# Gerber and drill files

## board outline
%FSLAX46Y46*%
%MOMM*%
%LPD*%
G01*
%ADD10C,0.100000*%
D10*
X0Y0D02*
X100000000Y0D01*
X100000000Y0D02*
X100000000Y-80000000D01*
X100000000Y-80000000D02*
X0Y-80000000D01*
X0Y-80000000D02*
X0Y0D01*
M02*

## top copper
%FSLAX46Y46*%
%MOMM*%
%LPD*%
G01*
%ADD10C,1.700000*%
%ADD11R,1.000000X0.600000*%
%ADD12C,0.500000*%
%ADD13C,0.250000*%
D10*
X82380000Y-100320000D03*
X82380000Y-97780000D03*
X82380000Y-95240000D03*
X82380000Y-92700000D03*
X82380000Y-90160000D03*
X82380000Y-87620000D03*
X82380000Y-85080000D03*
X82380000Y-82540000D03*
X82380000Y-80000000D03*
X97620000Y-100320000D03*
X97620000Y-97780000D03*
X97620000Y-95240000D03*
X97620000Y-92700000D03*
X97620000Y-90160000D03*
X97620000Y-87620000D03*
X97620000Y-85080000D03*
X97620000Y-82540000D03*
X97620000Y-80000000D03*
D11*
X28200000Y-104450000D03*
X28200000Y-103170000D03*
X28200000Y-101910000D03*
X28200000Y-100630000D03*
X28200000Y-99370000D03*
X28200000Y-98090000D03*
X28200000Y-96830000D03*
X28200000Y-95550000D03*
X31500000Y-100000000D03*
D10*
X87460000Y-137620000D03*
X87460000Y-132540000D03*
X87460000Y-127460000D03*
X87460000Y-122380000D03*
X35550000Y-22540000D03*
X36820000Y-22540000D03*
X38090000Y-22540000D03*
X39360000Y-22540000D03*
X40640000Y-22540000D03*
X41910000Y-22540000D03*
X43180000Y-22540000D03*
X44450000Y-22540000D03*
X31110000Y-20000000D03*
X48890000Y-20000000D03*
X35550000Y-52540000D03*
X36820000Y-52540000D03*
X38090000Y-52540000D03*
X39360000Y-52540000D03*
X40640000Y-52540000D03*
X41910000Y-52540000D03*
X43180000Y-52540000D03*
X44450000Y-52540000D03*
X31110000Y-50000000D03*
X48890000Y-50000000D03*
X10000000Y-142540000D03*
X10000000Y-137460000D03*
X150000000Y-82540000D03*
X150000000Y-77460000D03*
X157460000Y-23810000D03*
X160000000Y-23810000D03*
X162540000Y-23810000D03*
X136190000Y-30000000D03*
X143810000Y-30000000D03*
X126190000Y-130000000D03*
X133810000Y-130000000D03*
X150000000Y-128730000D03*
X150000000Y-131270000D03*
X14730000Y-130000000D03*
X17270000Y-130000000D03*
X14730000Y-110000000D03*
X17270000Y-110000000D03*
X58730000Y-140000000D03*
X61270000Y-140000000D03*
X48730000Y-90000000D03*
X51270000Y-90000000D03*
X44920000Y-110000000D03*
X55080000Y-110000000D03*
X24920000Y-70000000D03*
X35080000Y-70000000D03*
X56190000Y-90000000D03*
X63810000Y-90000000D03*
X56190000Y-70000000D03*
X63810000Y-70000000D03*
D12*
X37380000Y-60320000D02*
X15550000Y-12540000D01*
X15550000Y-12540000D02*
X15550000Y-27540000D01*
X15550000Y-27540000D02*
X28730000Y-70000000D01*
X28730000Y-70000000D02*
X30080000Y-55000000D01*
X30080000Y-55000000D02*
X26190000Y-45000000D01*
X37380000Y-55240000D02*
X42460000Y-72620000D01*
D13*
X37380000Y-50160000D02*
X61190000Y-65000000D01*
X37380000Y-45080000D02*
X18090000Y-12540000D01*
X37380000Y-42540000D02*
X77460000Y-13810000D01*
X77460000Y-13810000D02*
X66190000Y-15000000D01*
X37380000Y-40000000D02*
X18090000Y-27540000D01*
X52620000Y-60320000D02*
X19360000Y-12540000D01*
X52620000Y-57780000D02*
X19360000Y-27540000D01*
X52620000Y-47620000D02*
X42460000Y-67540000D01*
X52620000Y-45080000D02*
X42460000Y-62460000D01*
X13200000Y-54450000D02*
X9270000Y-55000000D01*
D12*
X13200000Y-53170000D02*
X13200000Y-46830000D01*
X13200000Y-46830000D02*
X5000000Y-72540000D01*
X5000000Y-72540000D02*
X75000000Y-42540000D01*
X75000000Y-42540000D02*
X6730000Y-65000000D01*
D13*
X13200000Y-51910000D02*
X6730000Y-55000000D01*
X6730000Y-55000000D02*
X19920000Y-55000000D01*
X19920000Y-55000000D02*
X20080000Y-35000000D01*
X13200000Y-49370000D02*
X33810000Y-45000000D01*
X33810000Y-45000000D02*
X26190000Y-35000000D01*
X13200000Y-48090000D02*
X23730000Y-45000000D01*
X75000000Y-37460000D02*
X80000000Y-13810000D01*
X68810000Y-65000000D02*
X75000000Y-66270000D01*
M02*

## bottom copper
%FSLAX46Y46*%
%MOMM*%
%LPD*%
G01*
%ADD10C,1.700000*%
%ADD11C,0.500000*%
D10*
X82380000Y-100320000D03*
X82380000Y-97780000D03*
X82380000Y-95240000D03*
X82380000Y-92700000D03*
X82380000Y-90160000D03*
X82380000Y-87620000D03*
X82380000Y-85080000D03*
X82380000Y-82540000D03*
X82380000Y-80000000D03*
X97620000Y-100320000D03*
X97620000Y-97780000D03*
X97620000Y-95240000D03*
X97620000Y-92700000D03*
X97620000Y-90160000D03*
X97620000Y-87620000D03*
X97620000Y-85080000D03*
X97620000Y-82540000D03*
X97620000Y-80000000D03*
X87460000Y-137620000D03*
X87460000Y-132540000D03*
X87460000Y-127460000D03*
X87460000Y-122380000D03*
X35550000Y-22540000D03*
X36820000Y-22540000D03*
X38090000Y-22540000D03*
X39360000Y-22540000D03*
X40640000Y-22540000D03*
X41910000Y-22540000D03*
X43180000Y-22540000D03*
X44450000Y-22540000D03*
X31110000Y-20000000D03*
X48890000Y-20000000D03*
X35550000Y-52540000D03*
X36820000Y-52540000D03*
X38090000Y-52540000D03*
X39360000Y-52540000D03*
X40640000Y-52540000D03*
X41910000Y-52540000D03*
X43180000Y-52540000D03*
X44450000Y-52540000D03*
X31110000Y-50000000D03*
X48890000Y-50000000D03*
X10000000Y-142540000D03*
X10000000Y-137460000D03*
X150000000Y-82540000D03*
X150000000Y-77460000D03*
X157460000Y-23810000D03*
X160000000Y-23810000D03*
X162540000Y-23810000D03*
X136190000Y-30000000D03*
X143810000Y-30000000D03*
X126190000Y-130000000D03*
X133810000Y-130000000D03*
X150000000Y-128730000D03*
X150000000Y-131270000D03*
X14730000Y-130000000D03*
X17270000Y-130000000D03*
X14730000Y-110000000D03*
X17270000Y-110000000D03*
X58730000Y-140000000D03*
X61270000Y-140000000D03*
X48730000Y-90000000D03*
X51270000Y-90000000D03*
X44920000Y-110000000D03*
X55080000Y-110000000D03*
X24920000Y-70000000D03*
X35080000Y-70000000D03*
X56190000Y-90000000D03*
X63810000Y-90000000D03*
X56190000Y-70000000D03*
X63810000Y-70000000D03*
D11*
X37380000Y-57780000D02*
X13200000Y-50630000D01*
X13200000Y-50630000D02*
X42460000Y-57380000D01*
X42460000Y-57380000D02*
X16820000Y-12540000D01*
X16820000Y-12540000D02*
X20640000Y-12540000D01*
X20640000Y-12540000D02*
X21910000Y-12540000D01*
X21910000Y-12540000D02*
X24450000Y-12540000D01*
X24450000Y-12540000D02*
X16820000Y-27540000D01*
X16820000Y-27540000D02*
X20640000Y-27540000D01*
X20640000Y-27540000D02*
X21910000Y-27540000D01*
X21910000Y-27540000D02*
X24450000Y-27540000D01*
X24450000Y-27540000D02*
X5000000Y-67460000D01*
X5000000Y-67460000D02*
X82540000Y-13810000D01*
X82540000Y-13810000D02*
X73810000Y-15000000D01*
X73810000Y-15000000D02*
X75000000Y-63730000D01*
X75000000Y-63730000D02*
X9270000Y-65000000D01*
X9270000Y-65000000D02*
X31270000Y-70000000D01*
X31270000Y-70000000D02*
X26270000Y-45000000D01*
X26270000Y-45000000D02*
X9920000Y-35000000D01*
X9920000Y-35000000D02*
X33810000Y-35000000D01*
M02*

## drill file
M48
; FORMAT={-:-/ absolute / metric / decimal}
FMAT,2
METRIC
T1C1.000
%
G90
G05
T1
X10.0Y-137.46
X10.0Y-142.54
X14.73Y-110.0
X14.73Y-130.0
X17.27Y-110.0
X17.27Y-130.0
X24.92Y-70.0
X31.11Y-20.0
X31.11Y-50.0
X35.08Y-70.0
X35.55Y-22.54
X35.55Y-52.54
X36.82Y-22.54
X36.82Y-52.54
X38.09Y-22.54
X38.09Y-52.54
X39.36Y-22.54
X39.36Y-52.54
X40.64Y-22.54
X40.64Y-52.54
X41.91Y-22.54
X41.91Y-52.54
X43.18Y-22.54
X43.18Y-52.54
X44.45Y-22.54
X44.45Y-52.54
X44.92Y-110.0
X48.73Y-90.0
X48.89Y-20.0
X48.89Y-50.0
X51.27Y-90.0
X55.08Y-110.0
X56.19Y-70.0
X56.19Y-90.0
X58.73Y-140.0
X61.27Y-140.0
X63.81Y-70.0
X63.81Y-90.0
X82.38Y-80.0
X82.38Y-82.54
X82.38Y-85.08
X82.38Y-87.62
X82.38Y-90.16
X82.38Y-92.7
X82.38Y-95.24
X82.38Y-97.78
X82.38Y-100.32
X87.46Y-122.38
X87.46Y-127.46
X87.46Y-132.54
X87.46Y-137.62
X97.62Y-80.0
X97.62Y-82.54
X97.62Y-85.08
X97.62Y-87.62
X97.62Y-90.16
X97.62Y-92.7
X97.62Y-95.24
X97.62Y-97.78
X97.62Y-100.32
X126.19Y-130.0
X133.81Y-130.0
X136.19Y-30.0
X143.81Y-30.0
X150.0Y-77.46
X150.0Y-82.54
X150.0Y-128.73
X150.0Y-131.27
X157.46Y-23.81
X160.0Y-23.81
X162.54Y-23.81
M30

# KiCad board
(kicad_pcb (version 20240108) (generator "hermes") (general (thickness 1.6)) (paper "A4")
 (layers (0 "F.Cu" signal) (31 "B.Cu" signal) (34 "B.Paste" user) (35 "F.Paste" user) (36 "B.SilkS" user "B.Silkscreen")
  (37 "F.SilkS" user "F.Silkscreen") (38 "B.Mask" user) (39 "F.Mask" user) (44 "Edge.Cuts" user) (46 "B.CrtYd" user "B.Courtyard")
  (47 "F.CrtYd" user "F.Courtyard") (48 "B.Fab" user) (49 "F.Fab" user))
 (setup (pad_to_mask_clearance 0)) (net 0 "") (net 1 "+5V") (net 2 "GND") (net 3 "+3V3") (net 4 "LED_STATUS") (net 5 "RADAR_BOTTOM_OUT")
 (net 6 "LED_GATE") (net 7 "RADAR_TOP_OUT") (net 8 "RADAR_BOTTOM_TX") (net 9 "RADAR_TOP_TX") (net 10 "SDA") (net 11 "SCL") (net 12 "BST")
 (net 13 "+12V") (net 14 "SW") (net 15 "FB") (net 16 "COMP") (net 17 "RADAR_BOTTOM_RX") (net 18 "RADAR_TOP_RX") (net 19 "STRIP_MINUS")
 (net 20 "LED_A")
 (gr_line (start 0 0) (end 100 0) (stroke (width 0.1) (type default)) (layer "Edge.Cuts"))
 (gr_line (start 100 0) (end 100 80) (stroke (width 0.1) (type default)) (layer "Edge.Cuts"))
 (gr_line (start 100 80) (end 0 80) (stroke (width 0.1) (type default)) (layer "Edge.Cuts"))
 (gr_line (start 0 80) (end 0 0) (stroke (width 0.1) (type default)) (layer "Edge.Cuts"))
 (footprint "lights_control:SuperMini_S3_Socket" (layer "F.Cu") (at 45 40 0) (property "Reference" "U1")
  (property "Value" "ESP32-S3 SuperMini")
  (pad "1" thru_hole circle (at 37.38 60.32) (size 1.7 1.7) (drill 1.0) (layers "*.Cu" "*.Mask") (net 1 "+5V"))
  (pad "2" thru_hole circle (at 37.38 57.78) (size 1.7 1.7) (drill 1.0) (layers "*.Cu" "*.Mask") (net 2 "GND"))
  (pad "3" thru_hole circle (at 37.38 55.24) (size 1.7 1.7) (drill 1.0) (layers "*.Cu" "*.Mask") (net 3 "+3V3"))
  (pad "4" thru_hole circle (at 37.38 52.70) (size 1.7 1.7) (drill 1.0) (layers "*.Cu" "*.Mask"))
  (pad "5" thru_hole circle (at 37.38 50.16) (size 1.7 1.7) (drill 1.0) (layers "*.Cu" "*.Mask") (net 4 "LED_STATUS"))
  (pad "6" thru_hole circle (at 37.38 47.62) (size 1.7 1.7) (drill 1.0) (layers "*.Cu" "*.Mask"))
  (pad "7" thru_hole circle (at 37.38 45.08) (size 1.7 1.7) (drill 1.0) (layers "*.Cu" "*.Mask") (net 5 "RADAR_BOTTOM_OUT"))
  (pad "8" thru_hole circle (at 37.38 42.54) (size 1.7 1.7) (drill 1.0) (layers "*.Cu" "*.Mask") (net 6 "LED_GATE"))
  (pad "9" thru_hole circle (at 37.38 40.00) (size 1.7 1.7) (drill 1.0) (layers "*.Cu" "*.Mask") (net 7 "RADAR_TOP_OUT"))
  (pad "10" thru_hole circle (at 52.62 60.32) (size 1.7 1.7) (drill 1.0) (layers "*.Cu" "*.Mask") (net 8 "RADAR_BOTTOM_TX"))
  (pad "11" thru_hole circle (at 52.62 57.78) (size 1.7 1.7) (drill 1.0) (layers "*.Cu" "*.Mask") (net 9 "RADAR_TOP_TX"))
  (pad "12" thru_hole circle (at 52.62 55.24) (size 1.7 1.7) (drill 1.0) (layers "*.Cu" "*.Mask"))
  (pad "13" thru_hole circle (at 52.62 52.70) (size 1.7 1.7) (drill 1.0) (layers "*.Cu" "*.Mask"))
  (pad "14" thru_hole circle (at 52.62 50.16) (size 1.7 1.7) (drill 1.0) (layers "*.Cu" "*.Mask"))
  (pad "15" thru_hole circle (at 52.62 47.62) (size 1.7 1.7) (drill 1.0) (layers "*.Cu" "*.Mask") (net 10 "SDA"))
  (pad "16" thru_hole circle (at 52.62 45.08) (size 1.7 1.7) (drill 1.0) (layers "*.Cu" "*.Mask") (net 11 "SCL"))
  (pad "17" thru_hole circle (at 52.62 42.54) (size 1.7 1.7) (drill 1.0) (layers "*.Cu" "*.Mask"))
  (pad "18" thru_hole circle (at 52.62 40.00) (size 1.7 1.7) (drill 1.0) (layers "*.Cu" "*.Mask")))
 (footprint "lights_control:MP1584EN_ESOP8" (layer "F.Cu") (at 15 50 0) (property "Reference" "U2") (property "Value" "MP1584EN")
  (pad "1" smd rect (at 13.20 54.45) (size 1.0 0.6) (layers "F.Cu" "F.Paste" "F.Mask") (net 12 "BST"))
  (pad "2" smd rect (at 13.20 53.17) (size 1.0 0.6) (layers "F.Cu" "F.Paste" "F.Mask") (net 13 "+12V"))
  (pad "3" smd rect (at 13.20 51.91) (size 1.0 0.6) (layers "F.Cu" "F.Paste" "F.Mask") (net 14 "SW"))
  (pad "4" smd rect (at 13.20 50.63) (size 1.0 0.6) (layers "F.Cu" "F.Paste" "F.Mask") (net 2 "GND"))
  (pad "5" smd rect (at 13.20 49.37) (size 1.0 0.6) (layers "F.Cu" "F.Paste" "F.Mask") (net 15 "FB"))
  (pad "6" smd rect (at 13.20 48.09) (size 1.0 0.6) (layers "F.Cu" "F.Paste" "F.Mask") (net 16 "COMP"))
  (pad "7" smd rect (at 13.20 46.83) (size 1.0 0.6) (layers "F.Cu" "F.Paste" "F.Mask") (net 13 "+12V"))
  (pad "8" smd rect (at 13.20 45.55) (size 1.0 0.6) (layers "F.Cu" "F.Paste" "F.Mask"))
  (pad "9" smd rect (at 16.50 50.00) (size 1.0 0.6) (layers "F.Cu" "F.Paste" "F.Mask")))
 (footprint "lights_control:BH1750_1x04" (layer "F.Cu") (at 45 65 0) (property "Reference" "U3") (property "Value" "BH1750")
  (pad "1" thru_hole circle (at 42.46 72.62) (size 1.7 1.7) (drill 1.0) (layers "*.Cu" "*.Mask") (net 3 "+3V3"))
  (pad "2" thru_hole circle (at 42.46 67.54) (size 1.7 1.7) (drill 1.0) (layers "*.Cu" "*.Mask") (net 10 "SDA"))
  (pad "3" thru_hole circle (at 42.46 62.46) (size 1.7 1.7) (drill 1.0) (layers "*.Cu" "*.Mask") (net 11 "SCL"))
  (pad "4" thru_hole circle (at 42.46 57.38) (size 1.7 1.7) (drill 1.0) (layers "*.Cu" "*.Mask") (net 2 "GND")))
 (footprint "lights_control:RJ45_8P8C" (layer "F.Cu") (at 20 10 0) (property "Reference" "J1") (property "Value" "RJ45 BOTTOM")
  (pad "1" thru_hole circle (at 15.55 12.54) (size 1.7 1.7) (drill 1.0) (layers "*.Cu" "*.Mask") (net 1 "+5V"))
  (pad "2" thru_hole circle (at 16.82 12.54) (size 1.7 1.7) (drill 1.0) (layers "*.Cu" "*.Mask") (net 2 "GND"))
  (pad "3" thru_hole circle (at 18.09 12.54) (size 1.7 1.7) (drill 1.0) (layers "*.Cu" "*.Mask") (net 5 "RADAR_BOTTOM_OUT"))
  (pad "4" thru_hole circle (at 19.36 12.54) (size 1.7 1.7) (drill 1.0) (layers "*.Cu" "*.Mask") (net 8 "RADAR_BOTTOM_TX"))
  (pad "5" thru_hole circle (at 20.64 12.54) (size 1.7 1.7) (drill 1.0) (layers "*.Cu" "*.Mask") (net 2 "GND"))
  (pad "6" thru_hole circle (at 21.91 12.54) (size 1.7 1.7) (drill 1.0) (layers "*.Cu" "*.Mask") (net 2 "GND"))
  (pad "7" thru_hole circle (at 23.18 12.54) (size 1.7 1.7) (drill 1.0) (layers "*.Cu" "*.Mask") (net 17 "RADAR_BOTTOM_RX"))
  (pad "8" thru_hole circle (at 24.45 12.54) (size 1.7 1.7) (drill 1.0) (layers "*.Cu" "*.Mask") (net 2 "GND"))
  (pad "S1" thru_hole circle (at 11.11 10.00) (size 1.7 1.7) (drill 1.0) (layers "*.Cu" "*.Mask"))
  (pad "S2" thru_hole circle (at 28.89 10.00) (size 1.7 1.7) (drill 1.0) (layers "*.Cu" "*.Mask")))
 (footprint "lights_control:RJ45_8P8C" (layer "F.Cu") (at 20 25 0) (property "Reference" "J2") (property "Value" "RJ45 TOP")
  (pad "1" thru_hole circle (at 15.55 27.54) (size 1.7 1.7) (drill 1.0) (layers "*.Cu" "*.Mask") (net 1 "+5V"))
  (pad "2" thru_hole circle (at 16.82 27.54) (size 1.7 1.7) (drill 1.0) (layers "*.Cu" "*.Mask") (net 2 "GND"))
  (pad "3" thru_hole circle (at 18.09 27.54) (size 1.7 1.7) (drill 1.0) (layers "*.Cu" "*.Mask") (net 7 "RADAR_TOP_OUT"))
  (pad "4" thru_hole circle (at 19.36 27.54) (size 1.7 1.7) (drill 1.0) (layers "*.Cu" "*.Mask") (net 9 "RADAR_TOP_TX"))
  (pad "5" thru_hole circle (at 20.64 27.54) (size 1.7 1.7) (drill 1.0) (layers "*.Cu" "*.Mask") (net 2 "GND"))
  (pad "6" thru_hole circle (at 21.91 27.54) (size 1.7 1.7) (drill 1.0) (layers "*.Cu" "*.Mask") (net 2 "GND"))
  (pad "7" thru_hole circle (at 23.18 27.54) (size 1.7 1.7) (drill 1.0) (layers "*.Cu" "*.Mask") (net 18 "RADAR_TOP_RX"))
  (pad "8" thru_hole circle (at 24.45 27.54) (size 1.7 1.7) (drill 1.0) (layers "*.Cu" "*.Mask") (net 2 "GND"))
  (pad "S1" thru_hole circle (at 11.11 25.00) (size 1.7 1.7) (drill 1.0) (layers "*.Cu" "*.Mask"))
  (pad "S2" thru_hole circle (at 28.89 25.00) (size 1.7 1.7) (drill 1.0) (layers "*.Cu" "*.Mask")))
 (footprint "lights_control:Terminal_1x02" (layer "F.Cu") (at 5 70 0) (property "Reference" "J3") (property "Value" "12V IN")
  (pad "1" thru_hole circle (at 5.00 72.54) (size 1.7 1.7) (drill 1.0) (layers "*.Cu" "*.Mask") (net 13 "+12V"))
  (pad "2" thru_hole circle (at 5.00 67.46) (size 1.7 1.7) (drill 1.0) (layers "*.Cu" "*.Mask") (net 2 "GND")))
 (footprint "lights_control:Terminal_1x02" (layer "F.Cu") (at 75 40 0) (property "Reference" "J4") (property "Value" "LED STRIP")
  (pad "1" thru_hole circle (at 75.00 42.54) (size 1.7 1.7) (drill 1.0) (layers "*.Cu" "*.Mask") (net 13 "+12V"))
  (pad "2" thru_hole circle (at 75.00 37.46) (size 1.7 1.7) (drill 1.0) (layers "*.Cu" "*.Mask") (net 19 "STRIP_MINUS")))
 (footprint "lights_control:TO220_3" (layer "F.Cu") (at 80 10 0) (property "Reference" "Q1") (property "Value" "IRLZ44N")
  (pad "1" thru_hole circle (at 77.46 13.81) (size 1.7 1.7) (drill 1.0) (layers "*.Cu" "*.Mask") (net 6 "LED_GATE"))
  (pad "2" thru_hole circle (at 80.00 13.81) (size 1.7 1.7) (drill 1.0) (layers "*.Cu" "*.Mask") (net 19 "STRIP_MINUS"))
  (pad "3" thru_hole circle (at 82.54 13.81) (size 1.7 1.7) (drill 1.0) (layers "*.Cu" "*.Mask") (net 2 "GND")))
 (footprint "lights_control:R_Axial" (layer "F.Cu") (at 70 15 0) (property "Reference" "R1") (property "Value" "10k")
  (pad "1" thru_hole circle (at 66.19 15.00) (size 1.7 1.7) (drill 1.0) (layers "*.Cu" "*.Mask") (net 6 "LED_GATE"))
  (pad "2" thru_hole circle (at 73.81 15.00) (size 1.7 1.7) (drill 1.0) (layers "*.Cu" "*.Mask") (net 2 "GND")))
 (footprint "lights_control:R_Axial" (layer "F.Cu") (at 65 65 0) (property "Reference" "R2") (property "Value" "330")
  (pad "1" thru_hole circle (at 61.19 65.00) (size 1.7 1.7) (drill 1.0) (layers "*.Cu" "*.Mask") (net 4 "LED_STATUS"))
  (pad "2" thru_hole circle (at 68.81 65.00) (size 1.7 1.7) (drill 1.0) (layers "*.Cu" "*.Mask") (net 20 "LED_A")))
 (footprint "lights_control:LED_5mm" (layer "F.Cu") (at 75 65 0) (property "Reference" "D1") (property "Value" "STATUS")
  (pad "1" thru_hole circle (at 75.00 63.73) (size 1.7 1.7) (drill 1.0) (layers "*.Cu" "*.Mask") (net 2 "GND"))
  (pad "2" thru_hole circle (at 75.00 66.27) (size 1.7 1.7) (drill 1.0) (layers "*.Cu" "*.Mask") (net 20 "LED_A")))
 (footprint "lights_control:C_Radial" (layer "F.Cu") (at 8 65 0) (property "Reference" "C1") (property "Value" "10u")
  (pad "1" thru_hole circle (at 6.73 65.00) (size 1.7 1.7) (drill 1.0) (layers "*.Cu" "*.Mask") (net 13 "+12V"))
  (pad "2" thru_hole circle (at 9.27 65.00) (size 1.7 1.7) (drill 1.0) (layers "*.Cu" "*.Mask") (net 2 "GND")))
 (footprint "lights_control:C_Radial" (layer "F.Cu") (at 8 55 0) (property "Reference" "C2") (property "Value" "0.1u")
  (pad "1" thru_hole circle (at 6.73 55.00) (size 1.7 1.7) (drill 1.0) (layers "*.Cu" "*.Mask") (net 14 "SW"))
  (pad "2" thru_hole circle (at 9.27 55.00) (size 1.7 1.7) (drill 1.0) (layers "*.Cu" "*.Mask") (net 12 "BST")))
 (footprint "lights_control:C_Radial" (layer "F.Cu") (at 30 70 0) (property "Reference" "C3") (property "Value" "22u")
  (pad "1" thru_hole circle (at 28.73 70.00) (size 1.7 1.7) (drill 1.0) (layers "*.Cu" "*.Mask") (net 1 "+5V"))
  (pad "2" thru_hole circle (at 31.27 70.00) (size 1.7 1.7) (drill 1.0) (layers "*.Cu" "*.Mask") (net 2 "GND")))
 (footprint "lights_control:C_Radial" (layer "F.Cu") (at 25 45 0) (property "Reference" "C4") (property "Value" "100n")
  (pad "1" thru_hole circle (at 23.73 45.00) (size 1.7 1.7) (drill 1.0) (layers "*.Cu" "*.Mask") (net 16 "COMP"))
  (pad "2" thru_hole circle (at 26.27 45.00) (size 1.7 1.7) (drill 1.0) (layers "*.Cu" "*.Mask") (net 2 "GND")))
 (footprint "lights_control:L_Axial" (layer "F.Cu") (at 25 55 0) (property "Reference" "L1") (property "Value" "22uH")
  (pad "1" thru_hole circle (at 19.92 55.00) (size 1.7 1.7) (drill 1.0) (layers "*.Cu" "*.Mask") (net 14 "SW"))
  (pad "2" thru_hole circle (at 30.08 55.00) (size 1.7 1.7) (drill 1.0) (layers "*.Cu" "*.Mask") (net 1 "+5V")))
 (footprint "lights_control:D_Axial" (layer "F.Cu") (at 15 35 0) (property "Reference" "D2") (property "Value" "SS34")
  (pad "1" thru_hole circle (at 9.92 35.00) (size 1.7 1.7) (drill 1.0) (layers "*.Cu" "*.Mask") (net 2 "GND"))
  (pad "2" thru_hole circle (at 20.08 35.00) (size 1.7 1.7) (drill 1.0) (layers "*.Cu" "*.Mask") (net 14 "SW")))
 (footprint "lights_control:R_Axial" (layer "F.Cu") (at 30 45 0) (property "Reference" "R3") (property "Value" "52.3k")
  (pad "1" thru_hole circle (at 26.19 45.00) (size 1.7 1.7) (drill 1.0) (layers "*.Cu" "*.Mask") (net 1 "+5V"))
  (pad "2" thru_hole circle (at 33.81 45.00) (size 1.7 1.7) (drill 1.0) (layers "*.Cu" "*.Mask") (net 15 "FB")))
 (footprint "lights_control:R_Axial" (layer "F.Cu") (at 30 35 0) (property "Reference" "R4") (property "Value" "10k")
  (pad "1" thru_hole circle (at 26.19 35.00) (size 1.7 1.7) (drill 1.0) (layers "*.Cu" "*.Mask") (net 15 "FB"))
  (pad "2" thru_hole circle (at 33.81 35.00) (size 1.7 1.7) (drill 1.0) (layers "*.Cu" "*.Mask") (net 2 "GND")))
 (segment (start 37.38 60.32) (end 15.55 12.54) (width 0.5) (layer "F.Cu") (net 1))
 (segment (start 15.55 12.54) (end 15.55 27.54) (width 0.5) (layer "F.Cu") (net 1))
 (segment (start 15.55 27.54) (end 28.73 70.00) (width 0.5) (layer "F.Cu") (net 1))
 (segment (start 28.73 70.00) (end 30.08 55.00) (width 0.5) (layer "F.Cu") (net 1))
 (segment (start 30.08 55.00) (end 26.19 45.00) (width 0.5) (layer "F.Cu") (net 1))
 (segment (start 37.38 57.78) (end 13.20 50.63) (width 0.5) (layer "B.Cu") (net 2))
 (segment (start 13.20 50.63) (end 42.46 57.38) (width 0.5) (layer "B.Cu") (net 2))
 (segment (start 42.46 57.38) (end 16.82 12.54) (width 0.5) (layer "B.Cu") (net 2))
 (segment (start 16.82 12.54) (end 20.64 12.54) (width 0.5) (layer "B.Cu") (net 2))
 (segment (start 20.64 12.54) (end 21.91 12.54) (width 0.5) (layer "B.Cu") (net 2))
 (segment (start 21.91 12.54) (end 24.45 12.54) (width 0.5) (layer "B.Cu") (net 2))
 (segment (start 24.45 12.54) (end 16.82 27.54) (width 0.5) (layer "B.Cu") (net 2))
 (segment (start 16.82 27.54) (end 20.64 27.54) (width 0.5) (layer "B.Cu") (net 2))
 (segment (start 20.64 27.54) (end 21.91 27.54) (width 0.5) (layer "B.Cu") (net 2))
 (segment (start 21.91 27.54) (end 24.45 27.54) (width 0.5) (layer "B.Cu") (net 2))
 (segment (start 24.45 27.54) (end 5.00 67.46) (width 0.5) (layer "B.Cu") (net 2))
 (segment (start 5.00 67.46) (end 82.54 13.81) (width 0.5) (layer "B.Cu") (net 2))
 (segment (start 82.54 13.81) (end 73.81 15.00) (width 0.5) (layer "B.Cu") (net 2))
 (segment (start 73.81 15.00) (end 75.00 63.73) (width 0.5) (layer "B.Cu") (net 2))
 (segment (start 75.00 63.73) (end 9.27 65.00) (width 0.5) (layer "B.Cu") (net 2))
 (segment (start 9.27 65.00) (end 31.27 70.00) (width 0.5) (layer "B.Cu") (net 2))
 (segment (start 31.27 70.00) (end 26.27 45.00) (width 0.5) (layer "B.Cu") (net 2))
 (segment (start 26.27 45.00) (end 9.92 35.00) (width 0.5) (layer "B.Cu") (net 2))
 (segment (start 9.92 35.00) (end 33.81 35.00) (width 0.5) (layer "B.Cu") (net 2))
 (segment (start 37.38 55.24) (end 42.46 72.62) (width 0.5) (layer "F.Cu") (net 3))
 (segment (start 37.38 50.16) (end 61.19 65.00) (width 0.25) (layer "F.Cu") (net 4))
 (segment (start 37.38 45.08) (end 18.09 12.54) (width 0.25) (layer "F.Cu") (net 5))
 (segment (start 37.38 42.54) (end 77.46 13.81) (width 0.25) (layer "F.Cu") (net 6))
 (segment (start 77.46 13.81) (end 66.19 15.00) (width 0.25) (layer "F.Cu") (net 6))
 (segment (start 37.38 40.00) (end 18.09 27.54) (width 0.25) (layer "F.Cu") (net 7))
 (segment (start 52.62 60.32) (end 19.36 12.54) (width 0.25) (layer "F.Cu") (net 8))
 (segment (start 52.62 57.78) (end 19.36 27.54) (width 0.25) (layer "F.Cu") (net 9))
 (segment (start 52.62 47.62) (end 42.46 67.54) (width 0.25) (layer "F.Cu") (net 10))
 (segment (start 52.62 45.08) (end 42.46 62.46) (width 0.25) (layer "F.Cu") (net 11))
 (segment (start 13.20 54.45) (end 9.27 55.00) (width 0.25) (layer "F.Cu") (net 12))
 (segment (start 13.20 53.17) (end 13.20 46.83) (width 0.5) (layer "F.Cu") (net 13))
 (segment (start 13.20 46.83) (end 5.00 72.54) (width 0.5) (layer "F.Cu") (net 13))
 (segment (start 5.00 72.54) (end 75.00 42.54) (width 0.5) (layer "F.Cu") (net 13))
 (segment (start 75.00 42.54) (end 6.73 65.00) (width 0.5) (layer "F.Cu") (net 13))
 (segment (start 13.20 51.91) (end 6.73 55.00) (width 0.25) (layer "F.Cu") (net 14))
 (segment (start 6.73 55.00) (end 19.92 55.00) (width 0.25) (layer "F.Cu") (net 14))
 (segment (start 19.92 55.00) (end 20.08 35.00) (width 0.25) (layer "F.Cu") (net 14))
 (segment (start 13.20 49.37) (end 33.81 45.00) (width 0.25) (layer "F.Cu") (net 15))
 (segment (start 33.81 45.00) (end 26.19 35.00) (width 0.25) (layer "F.Cu") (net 15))
 (segment (start 13.20 48.09) (end 23.73 45.00) (width 0.25) (layer "F.Cu") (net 16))
 (segment (start 75.00 37.46) (end 80.00 13.81) (width 0.25) (layer "F.Cu") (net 19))
 (segment (start 68.81 65.00) (end 75.00 66.27) (width 0.25) (layer "F.Cu") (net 20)))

